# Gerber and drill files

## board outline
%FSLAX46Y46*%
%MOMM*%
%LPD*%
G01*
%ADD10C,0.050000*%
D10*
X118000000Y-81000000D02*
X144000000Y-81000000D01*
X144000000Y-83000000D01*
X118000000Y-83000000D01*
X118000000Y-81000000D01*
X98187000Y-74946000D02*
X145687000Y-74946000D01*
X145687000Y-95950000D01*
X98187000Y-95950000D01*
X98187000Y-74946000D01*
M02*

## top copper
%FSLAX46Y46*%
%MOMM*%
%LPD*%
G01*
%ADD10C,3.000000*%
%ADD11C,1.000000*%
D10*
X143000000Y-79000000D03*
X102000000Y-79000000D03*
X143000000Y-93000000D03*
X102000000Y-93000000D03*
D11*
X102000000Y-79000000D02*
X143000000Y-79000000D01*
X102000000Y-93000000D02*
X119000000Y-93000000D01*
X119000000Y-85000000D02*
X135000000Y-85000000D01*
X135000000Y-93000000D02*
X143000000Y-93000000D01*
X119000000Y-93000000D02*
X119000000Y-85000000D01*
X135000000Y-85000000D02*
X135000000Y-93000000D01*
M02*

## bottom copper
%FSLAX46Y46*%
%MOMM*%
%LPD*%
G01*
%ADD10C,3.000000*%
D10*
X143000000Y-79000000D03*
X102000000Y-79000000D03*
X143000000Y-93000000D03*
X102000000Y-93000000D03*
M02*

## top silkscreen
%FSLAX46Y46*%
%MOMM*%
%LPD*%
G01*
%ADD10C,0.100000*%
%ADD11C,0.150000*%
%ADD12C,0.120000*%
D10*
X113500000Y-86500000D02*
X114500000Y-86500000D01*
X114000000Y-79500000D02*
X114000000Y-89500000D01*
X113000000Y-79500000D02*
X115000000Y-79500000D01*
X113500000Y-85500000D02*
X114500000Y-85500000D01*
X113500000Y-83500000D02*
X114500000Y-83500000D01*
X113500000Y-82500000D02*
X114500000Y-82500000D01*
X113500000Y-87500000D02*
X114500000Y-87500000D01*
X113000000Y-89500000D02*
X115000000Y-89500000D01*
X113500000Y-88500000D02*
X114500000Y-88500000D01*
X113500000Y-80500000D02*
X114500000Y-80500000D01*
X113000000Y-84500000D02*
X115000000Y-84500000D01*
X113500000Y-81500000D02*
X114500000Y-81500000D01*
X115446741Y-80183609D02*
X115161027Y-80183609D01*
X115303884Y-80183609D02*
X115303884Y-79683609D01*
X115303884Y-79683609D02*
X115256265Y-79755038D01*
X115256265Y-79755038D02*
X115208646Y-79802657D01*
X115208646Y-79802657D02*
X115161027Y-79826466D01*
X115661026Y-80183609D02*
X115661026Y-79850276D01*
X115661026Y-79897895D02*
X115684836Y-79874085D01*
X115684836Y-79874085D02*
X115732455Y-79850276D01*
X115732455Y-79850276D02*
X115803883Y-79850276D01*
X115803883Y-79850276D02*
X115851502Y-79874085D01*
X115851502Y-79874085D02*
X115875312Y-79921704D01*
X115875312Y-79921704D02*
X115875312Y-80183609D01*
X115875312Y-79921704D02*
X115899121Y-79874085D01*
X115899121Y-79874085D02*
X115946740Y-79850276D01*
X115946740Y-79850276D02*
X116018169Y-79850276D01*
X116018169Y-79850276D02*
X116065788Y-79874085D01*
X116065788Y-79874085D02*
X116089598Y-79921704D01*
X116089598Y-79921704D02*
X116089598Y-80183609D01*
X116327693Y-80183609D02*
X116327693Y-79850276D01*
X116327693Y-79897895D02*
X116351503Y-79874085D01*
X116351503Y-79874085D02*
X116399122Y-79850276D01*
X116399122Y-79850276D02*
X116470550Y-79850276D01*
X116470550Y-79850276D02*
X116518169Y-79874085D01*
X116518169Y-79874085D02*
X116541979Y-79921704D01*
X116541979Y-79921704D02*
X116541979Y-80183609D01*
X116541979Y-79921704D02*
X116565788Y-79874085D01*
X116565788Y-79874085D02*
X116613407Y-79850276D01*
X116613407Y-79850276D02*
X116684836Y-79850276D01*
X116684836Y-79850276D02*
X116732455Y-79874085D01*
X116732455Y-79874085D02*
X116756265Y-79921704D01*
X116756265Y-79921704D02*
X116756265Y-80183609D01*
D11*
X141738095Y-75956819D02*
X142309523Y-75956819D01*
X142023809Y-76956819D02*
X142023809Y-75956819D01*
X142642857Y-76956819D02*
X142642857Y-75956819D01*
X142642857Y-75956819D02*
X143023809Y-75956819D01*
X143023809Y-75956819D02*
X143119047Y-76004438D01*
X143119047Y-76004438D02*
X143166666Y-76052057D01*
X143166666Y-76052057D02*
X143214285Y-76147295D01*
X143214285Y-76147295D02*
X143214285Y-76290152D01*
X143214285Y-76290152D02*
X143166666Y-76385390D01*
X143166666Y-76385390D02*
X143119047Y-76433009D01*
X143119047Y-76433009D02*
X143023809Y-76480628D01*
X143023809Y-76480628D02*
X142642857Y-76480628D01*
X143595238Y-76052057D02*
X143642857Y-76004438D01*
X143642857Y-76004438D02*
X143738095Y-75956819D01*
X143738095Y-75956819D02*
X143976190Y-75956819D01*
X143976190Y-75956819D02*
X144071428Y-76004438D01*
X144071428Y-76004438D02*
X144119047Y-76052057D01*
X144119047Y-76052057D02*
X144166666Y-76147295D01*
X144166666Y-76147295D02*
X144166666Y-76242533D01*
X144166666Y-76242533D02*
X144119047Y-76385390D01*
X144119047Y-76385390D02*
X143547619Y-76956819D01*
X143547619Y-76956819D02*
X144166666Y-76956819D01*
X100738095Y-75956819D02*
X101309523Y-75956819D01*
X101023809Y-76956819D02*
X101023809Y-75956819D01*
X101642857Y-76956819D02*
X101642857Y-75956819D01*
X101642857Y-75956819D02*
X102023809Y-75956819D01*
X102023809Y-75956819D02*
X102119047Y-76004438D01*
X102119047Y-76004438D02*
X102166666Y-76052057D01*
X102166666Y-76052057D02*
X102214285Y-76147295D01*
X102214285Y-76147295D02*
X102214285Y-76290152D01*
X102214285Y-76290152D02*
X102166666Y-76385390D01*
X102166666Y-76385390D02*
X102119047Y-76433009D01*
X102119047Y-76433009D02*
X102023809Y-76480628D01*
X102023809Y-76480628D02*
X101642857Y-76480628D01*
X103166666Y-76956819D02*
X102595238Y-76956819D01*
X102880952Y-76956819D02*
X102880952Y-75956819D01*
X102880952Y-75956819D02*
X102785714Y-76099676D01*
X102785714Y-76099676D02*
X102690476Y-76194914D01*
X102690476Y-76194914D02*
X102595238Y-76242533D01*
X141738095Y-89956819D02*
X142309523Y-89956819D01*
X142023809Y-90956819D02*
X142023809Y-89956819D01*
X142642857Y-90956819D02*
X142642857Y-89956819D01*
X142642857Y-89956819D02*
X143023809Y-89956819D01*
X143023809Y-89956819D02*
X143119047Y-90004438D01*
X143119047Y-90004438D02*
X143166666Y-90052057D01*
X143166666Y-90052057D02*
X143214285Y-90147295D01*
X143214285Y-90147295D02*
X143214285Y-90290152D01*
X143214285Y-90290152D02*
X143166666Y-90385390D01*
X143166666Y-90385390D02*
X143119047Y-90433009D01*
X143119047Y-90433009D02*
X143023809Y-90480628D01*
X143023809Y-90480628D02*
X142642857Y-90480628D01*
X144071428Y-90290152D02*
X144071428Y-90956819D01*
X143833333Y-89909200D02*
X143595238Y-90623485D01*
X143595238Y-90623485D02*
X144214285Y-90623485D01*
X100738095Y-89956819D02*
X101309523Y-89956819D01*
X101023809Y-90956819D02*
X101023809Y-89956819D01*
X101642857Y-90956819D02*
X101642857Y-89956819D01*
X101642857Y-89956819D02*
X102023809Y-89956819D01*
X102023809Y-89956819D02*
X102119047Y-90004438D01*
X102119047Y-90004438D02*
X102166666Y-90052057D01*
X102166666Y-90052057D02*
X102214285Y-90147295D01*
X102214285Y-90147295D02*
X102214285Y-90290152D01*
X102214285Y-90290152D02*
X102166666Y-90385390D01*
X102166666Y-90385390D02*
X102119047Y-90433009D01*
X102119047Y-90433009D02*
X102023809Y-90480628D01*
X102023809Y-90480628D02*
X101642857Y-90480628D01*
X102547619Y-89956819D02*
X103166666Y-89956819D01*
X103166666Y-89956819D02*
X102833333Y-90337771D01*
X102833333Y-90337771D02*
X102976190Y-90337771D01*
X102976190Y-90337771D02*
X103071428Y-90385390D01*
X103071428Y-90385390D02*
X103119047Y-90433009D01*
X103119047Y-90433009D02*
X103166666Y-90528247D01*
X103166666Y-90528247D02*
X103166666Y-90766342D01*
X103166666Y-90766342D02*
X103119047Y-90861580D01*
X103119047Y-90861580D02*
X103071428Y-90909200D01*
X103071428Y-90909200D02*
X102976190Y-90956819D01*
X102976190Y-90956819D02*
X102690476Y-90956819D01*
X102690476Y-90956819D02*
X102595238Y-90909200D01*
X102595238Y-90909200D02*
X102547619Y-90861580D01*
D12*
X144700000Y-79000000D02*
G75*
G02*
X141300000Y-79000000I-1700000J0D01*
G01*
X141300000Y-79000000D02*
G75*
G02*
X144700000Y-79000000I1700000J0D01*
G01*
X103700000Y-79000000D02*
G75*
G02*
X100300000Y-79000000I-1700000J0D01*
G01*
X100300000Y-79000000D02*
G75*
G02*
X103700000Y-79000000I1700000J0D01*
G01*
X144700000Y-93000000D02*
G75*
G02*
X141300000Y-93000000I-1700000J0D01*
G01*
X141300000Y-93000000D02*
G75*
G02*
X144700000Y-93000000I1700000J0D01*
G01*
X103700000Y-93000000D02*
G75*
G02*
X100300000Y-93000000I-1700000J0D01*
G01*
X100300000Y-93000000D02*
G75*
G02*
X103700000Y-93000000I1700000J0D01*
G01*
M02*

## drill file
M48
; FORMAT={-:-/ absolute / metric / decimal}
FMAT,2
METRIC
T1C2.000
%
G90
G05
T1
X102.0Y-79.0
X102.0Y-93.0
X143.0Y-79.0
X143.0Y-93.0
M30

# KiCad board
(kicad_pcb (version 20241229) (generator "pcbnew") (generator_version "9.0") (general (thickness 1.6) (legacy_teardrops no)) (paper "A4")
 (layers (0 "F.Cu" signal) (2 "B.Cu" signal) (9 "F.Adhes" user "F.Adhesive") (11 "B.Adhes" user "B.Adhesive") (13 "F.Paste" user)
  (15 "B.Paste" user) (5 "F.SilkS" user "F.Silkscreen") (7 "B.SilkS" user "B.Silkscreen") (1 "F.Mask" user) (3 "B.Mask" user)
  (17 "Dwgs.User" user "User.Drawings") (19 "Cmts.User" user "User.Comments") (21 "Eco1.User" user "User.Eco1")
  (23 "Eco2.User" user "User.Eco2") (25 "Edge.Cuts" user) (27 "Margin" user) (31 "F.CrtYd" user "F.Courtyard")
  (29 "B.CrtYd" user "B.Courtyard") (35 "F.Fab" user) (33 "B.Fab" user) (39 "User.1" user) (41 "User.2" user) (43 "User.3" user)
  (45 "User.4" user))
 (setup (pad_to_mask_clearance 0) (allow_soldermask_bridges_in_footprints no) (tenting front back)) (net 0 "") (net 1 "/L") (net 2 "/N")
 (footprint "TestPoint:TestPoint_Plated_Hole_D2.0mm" (layer "F.Cu") (at 143 79)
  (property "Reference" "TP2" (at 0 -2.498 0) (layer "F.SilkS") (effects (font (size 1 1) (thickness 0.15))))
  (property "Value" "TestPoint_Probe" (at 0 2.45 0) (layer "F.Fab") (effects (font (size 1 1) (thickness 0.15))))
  (fp_circle (center 0 0) (end 0 -1.7) (stroke (width 0.12) (type solid)) (fill no) (layer "F.SilkS"))
  (pad "1" thru_hole circle (at 0 0) (size 3 3) (drill 2) (layers "*.Cu" "*.Mask") (remove_unused_layers no) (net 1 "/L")))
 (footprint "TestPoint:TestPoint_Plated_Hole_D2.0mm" (layer "F.Cu") (at 102 79)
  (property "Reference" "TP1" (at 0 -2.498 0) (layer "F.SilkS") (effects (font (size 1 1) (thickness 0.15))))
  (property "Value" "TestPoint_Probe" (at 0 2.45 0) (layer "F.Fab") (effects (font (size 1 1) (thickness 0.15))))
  (fp_circle (center 0 0) (end 0 -1.7) (stroke (width 0.12) (type solid)) (fill no) (layer "F.SilkS"))
  (pad "1" thru_hole circle (at 0 0) (size 3 3) (drill 2) (layers "*.Cu" "*.Mask") (remove_unused_layers no) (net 1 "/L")))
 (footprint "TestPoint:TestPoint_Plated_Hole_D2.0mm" (layer "F.Cu") (at 143 93)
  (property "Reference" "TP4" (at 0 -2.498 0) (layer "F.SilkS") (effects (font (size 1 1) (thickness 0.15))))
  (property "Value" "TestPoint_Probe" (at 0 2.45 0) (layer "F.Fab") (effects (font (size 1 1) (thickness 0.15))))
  (fp_circle (center 0 0) (end 0 -1.7) (stroke (width 0.12) (type solid)) (fill no) (layer "F.SilkS"))
  (pad "1" thru_hole circle (at 0 0) (size 3 3) (drill 2) (layers "*.Cu" "*.Mask") (remove_unused_layers no) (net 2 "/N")))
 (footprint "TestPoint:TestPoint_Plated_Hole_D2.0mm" (layer "F.Cu") (at 102 93)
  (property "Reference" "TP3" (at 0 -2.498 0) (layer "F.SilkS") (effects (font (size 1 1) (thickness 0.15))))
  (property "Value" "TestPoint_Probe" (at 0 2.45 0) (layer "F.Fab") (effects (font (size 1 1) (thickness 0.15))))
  (fp_circle (center 0 0) (end 0 -1.7) (stroke (width 0.12) (type solid)) (fill no) (layer "F.SilkS"))
  (pad "1" thru_hole circle (at 0 0) (size 3 3) (drill 2) (layers "*.Cu" "*.Mask") (remove_unused_layers no) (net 2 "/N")))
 (gr_line (start 113.5 86.5) (end 114.5 86.5) (stroke (width 0.1) (type default)) (layer "F.SilkS"))
 (gr_line (start 114 79.5) (end 114 89.5) (stroke (width 0.1) (type default)) (layer "F.SilkS"))
 (gr_line (start 113 79.5) (end 115 79.5) (stroke (width 0.1) (type default)) (layer "F.SilkS"))
 (gr_line (start 113.5 85.5) (end 114.5 85.5) (stroke (width 0.1) (type default)) (layer "F.SilkS"))
 (gr_line (start 113.5 83.5) (end 114.5 83.5) (stroke (width 0.1) (type default)) (layer "F.SilkS"))
 (gr_line (start 113.5 82.5) (end 114.5 82.5) (stroke (width 0.1) (type default)) (layer "F.SilkS"))
 (gr_line (start 113.5 87.5) (end 114.5 87.5) (stroke (width 0.1) (type default)) (layer "F.SilkS"))
 (gr_line (start 113 89.5) (end 115 89.5) (stroke (width 0.1) (type default)) (layer "F.SilkS"))
 (gr_line (start 113.5 88.5) (end 114.5 88.5) (stroke (width 0.1) (type default)) (layer "F.SilkS"))
 (gr_line (start 113.5 80.5) (end 114.5 80.5) (stroke (width 0.1) (type default)) (layer "F.SilkS"))
 (gr_line (start 113 84.5) (end 115 84.5) (stroke (width 0.1) (type default)) (layer "F.SilkS"))
 (gr_line (start 113.5 81.5) (end 114.5 81.5) (stroke (width 0.1) (type default)) (layer "F.SilkS"))
 (gr_rect (start 118 81) (end 144 83) (stroke (width 0.05) (type default)) (fill no) (layer "Edge.Cuts"))
 (gr_rect (start 98.187 74.946) (end 145.687 95.95) (stroke (width 0.05) (type default)) (fill no) (layer "Edge.Cuts"))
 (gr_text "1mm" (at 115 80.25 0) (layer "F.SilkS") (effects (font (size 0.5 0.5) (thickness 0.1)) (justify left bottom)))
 (segment (start 102 79) (end 143 79) (width 1) (layer "F.Cu") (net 1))
 (segment (start 102 93) (end 119 93) (width 1) (layer "F.Cu") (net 2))
 (segment (start 119 85) (end 135 85) (width 1) (layer "F.Cu") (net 2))
 (segment (start 135 93) (end 143 93) (width 1) (layer "F.Cu") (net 2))
 (segment (start 119 93) (end 119 85) (width 1) (layer "F.Cu") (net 2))
 (segment (start 135 85) (end 135 93) (width 1) (layer "F.Cu") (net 2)))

